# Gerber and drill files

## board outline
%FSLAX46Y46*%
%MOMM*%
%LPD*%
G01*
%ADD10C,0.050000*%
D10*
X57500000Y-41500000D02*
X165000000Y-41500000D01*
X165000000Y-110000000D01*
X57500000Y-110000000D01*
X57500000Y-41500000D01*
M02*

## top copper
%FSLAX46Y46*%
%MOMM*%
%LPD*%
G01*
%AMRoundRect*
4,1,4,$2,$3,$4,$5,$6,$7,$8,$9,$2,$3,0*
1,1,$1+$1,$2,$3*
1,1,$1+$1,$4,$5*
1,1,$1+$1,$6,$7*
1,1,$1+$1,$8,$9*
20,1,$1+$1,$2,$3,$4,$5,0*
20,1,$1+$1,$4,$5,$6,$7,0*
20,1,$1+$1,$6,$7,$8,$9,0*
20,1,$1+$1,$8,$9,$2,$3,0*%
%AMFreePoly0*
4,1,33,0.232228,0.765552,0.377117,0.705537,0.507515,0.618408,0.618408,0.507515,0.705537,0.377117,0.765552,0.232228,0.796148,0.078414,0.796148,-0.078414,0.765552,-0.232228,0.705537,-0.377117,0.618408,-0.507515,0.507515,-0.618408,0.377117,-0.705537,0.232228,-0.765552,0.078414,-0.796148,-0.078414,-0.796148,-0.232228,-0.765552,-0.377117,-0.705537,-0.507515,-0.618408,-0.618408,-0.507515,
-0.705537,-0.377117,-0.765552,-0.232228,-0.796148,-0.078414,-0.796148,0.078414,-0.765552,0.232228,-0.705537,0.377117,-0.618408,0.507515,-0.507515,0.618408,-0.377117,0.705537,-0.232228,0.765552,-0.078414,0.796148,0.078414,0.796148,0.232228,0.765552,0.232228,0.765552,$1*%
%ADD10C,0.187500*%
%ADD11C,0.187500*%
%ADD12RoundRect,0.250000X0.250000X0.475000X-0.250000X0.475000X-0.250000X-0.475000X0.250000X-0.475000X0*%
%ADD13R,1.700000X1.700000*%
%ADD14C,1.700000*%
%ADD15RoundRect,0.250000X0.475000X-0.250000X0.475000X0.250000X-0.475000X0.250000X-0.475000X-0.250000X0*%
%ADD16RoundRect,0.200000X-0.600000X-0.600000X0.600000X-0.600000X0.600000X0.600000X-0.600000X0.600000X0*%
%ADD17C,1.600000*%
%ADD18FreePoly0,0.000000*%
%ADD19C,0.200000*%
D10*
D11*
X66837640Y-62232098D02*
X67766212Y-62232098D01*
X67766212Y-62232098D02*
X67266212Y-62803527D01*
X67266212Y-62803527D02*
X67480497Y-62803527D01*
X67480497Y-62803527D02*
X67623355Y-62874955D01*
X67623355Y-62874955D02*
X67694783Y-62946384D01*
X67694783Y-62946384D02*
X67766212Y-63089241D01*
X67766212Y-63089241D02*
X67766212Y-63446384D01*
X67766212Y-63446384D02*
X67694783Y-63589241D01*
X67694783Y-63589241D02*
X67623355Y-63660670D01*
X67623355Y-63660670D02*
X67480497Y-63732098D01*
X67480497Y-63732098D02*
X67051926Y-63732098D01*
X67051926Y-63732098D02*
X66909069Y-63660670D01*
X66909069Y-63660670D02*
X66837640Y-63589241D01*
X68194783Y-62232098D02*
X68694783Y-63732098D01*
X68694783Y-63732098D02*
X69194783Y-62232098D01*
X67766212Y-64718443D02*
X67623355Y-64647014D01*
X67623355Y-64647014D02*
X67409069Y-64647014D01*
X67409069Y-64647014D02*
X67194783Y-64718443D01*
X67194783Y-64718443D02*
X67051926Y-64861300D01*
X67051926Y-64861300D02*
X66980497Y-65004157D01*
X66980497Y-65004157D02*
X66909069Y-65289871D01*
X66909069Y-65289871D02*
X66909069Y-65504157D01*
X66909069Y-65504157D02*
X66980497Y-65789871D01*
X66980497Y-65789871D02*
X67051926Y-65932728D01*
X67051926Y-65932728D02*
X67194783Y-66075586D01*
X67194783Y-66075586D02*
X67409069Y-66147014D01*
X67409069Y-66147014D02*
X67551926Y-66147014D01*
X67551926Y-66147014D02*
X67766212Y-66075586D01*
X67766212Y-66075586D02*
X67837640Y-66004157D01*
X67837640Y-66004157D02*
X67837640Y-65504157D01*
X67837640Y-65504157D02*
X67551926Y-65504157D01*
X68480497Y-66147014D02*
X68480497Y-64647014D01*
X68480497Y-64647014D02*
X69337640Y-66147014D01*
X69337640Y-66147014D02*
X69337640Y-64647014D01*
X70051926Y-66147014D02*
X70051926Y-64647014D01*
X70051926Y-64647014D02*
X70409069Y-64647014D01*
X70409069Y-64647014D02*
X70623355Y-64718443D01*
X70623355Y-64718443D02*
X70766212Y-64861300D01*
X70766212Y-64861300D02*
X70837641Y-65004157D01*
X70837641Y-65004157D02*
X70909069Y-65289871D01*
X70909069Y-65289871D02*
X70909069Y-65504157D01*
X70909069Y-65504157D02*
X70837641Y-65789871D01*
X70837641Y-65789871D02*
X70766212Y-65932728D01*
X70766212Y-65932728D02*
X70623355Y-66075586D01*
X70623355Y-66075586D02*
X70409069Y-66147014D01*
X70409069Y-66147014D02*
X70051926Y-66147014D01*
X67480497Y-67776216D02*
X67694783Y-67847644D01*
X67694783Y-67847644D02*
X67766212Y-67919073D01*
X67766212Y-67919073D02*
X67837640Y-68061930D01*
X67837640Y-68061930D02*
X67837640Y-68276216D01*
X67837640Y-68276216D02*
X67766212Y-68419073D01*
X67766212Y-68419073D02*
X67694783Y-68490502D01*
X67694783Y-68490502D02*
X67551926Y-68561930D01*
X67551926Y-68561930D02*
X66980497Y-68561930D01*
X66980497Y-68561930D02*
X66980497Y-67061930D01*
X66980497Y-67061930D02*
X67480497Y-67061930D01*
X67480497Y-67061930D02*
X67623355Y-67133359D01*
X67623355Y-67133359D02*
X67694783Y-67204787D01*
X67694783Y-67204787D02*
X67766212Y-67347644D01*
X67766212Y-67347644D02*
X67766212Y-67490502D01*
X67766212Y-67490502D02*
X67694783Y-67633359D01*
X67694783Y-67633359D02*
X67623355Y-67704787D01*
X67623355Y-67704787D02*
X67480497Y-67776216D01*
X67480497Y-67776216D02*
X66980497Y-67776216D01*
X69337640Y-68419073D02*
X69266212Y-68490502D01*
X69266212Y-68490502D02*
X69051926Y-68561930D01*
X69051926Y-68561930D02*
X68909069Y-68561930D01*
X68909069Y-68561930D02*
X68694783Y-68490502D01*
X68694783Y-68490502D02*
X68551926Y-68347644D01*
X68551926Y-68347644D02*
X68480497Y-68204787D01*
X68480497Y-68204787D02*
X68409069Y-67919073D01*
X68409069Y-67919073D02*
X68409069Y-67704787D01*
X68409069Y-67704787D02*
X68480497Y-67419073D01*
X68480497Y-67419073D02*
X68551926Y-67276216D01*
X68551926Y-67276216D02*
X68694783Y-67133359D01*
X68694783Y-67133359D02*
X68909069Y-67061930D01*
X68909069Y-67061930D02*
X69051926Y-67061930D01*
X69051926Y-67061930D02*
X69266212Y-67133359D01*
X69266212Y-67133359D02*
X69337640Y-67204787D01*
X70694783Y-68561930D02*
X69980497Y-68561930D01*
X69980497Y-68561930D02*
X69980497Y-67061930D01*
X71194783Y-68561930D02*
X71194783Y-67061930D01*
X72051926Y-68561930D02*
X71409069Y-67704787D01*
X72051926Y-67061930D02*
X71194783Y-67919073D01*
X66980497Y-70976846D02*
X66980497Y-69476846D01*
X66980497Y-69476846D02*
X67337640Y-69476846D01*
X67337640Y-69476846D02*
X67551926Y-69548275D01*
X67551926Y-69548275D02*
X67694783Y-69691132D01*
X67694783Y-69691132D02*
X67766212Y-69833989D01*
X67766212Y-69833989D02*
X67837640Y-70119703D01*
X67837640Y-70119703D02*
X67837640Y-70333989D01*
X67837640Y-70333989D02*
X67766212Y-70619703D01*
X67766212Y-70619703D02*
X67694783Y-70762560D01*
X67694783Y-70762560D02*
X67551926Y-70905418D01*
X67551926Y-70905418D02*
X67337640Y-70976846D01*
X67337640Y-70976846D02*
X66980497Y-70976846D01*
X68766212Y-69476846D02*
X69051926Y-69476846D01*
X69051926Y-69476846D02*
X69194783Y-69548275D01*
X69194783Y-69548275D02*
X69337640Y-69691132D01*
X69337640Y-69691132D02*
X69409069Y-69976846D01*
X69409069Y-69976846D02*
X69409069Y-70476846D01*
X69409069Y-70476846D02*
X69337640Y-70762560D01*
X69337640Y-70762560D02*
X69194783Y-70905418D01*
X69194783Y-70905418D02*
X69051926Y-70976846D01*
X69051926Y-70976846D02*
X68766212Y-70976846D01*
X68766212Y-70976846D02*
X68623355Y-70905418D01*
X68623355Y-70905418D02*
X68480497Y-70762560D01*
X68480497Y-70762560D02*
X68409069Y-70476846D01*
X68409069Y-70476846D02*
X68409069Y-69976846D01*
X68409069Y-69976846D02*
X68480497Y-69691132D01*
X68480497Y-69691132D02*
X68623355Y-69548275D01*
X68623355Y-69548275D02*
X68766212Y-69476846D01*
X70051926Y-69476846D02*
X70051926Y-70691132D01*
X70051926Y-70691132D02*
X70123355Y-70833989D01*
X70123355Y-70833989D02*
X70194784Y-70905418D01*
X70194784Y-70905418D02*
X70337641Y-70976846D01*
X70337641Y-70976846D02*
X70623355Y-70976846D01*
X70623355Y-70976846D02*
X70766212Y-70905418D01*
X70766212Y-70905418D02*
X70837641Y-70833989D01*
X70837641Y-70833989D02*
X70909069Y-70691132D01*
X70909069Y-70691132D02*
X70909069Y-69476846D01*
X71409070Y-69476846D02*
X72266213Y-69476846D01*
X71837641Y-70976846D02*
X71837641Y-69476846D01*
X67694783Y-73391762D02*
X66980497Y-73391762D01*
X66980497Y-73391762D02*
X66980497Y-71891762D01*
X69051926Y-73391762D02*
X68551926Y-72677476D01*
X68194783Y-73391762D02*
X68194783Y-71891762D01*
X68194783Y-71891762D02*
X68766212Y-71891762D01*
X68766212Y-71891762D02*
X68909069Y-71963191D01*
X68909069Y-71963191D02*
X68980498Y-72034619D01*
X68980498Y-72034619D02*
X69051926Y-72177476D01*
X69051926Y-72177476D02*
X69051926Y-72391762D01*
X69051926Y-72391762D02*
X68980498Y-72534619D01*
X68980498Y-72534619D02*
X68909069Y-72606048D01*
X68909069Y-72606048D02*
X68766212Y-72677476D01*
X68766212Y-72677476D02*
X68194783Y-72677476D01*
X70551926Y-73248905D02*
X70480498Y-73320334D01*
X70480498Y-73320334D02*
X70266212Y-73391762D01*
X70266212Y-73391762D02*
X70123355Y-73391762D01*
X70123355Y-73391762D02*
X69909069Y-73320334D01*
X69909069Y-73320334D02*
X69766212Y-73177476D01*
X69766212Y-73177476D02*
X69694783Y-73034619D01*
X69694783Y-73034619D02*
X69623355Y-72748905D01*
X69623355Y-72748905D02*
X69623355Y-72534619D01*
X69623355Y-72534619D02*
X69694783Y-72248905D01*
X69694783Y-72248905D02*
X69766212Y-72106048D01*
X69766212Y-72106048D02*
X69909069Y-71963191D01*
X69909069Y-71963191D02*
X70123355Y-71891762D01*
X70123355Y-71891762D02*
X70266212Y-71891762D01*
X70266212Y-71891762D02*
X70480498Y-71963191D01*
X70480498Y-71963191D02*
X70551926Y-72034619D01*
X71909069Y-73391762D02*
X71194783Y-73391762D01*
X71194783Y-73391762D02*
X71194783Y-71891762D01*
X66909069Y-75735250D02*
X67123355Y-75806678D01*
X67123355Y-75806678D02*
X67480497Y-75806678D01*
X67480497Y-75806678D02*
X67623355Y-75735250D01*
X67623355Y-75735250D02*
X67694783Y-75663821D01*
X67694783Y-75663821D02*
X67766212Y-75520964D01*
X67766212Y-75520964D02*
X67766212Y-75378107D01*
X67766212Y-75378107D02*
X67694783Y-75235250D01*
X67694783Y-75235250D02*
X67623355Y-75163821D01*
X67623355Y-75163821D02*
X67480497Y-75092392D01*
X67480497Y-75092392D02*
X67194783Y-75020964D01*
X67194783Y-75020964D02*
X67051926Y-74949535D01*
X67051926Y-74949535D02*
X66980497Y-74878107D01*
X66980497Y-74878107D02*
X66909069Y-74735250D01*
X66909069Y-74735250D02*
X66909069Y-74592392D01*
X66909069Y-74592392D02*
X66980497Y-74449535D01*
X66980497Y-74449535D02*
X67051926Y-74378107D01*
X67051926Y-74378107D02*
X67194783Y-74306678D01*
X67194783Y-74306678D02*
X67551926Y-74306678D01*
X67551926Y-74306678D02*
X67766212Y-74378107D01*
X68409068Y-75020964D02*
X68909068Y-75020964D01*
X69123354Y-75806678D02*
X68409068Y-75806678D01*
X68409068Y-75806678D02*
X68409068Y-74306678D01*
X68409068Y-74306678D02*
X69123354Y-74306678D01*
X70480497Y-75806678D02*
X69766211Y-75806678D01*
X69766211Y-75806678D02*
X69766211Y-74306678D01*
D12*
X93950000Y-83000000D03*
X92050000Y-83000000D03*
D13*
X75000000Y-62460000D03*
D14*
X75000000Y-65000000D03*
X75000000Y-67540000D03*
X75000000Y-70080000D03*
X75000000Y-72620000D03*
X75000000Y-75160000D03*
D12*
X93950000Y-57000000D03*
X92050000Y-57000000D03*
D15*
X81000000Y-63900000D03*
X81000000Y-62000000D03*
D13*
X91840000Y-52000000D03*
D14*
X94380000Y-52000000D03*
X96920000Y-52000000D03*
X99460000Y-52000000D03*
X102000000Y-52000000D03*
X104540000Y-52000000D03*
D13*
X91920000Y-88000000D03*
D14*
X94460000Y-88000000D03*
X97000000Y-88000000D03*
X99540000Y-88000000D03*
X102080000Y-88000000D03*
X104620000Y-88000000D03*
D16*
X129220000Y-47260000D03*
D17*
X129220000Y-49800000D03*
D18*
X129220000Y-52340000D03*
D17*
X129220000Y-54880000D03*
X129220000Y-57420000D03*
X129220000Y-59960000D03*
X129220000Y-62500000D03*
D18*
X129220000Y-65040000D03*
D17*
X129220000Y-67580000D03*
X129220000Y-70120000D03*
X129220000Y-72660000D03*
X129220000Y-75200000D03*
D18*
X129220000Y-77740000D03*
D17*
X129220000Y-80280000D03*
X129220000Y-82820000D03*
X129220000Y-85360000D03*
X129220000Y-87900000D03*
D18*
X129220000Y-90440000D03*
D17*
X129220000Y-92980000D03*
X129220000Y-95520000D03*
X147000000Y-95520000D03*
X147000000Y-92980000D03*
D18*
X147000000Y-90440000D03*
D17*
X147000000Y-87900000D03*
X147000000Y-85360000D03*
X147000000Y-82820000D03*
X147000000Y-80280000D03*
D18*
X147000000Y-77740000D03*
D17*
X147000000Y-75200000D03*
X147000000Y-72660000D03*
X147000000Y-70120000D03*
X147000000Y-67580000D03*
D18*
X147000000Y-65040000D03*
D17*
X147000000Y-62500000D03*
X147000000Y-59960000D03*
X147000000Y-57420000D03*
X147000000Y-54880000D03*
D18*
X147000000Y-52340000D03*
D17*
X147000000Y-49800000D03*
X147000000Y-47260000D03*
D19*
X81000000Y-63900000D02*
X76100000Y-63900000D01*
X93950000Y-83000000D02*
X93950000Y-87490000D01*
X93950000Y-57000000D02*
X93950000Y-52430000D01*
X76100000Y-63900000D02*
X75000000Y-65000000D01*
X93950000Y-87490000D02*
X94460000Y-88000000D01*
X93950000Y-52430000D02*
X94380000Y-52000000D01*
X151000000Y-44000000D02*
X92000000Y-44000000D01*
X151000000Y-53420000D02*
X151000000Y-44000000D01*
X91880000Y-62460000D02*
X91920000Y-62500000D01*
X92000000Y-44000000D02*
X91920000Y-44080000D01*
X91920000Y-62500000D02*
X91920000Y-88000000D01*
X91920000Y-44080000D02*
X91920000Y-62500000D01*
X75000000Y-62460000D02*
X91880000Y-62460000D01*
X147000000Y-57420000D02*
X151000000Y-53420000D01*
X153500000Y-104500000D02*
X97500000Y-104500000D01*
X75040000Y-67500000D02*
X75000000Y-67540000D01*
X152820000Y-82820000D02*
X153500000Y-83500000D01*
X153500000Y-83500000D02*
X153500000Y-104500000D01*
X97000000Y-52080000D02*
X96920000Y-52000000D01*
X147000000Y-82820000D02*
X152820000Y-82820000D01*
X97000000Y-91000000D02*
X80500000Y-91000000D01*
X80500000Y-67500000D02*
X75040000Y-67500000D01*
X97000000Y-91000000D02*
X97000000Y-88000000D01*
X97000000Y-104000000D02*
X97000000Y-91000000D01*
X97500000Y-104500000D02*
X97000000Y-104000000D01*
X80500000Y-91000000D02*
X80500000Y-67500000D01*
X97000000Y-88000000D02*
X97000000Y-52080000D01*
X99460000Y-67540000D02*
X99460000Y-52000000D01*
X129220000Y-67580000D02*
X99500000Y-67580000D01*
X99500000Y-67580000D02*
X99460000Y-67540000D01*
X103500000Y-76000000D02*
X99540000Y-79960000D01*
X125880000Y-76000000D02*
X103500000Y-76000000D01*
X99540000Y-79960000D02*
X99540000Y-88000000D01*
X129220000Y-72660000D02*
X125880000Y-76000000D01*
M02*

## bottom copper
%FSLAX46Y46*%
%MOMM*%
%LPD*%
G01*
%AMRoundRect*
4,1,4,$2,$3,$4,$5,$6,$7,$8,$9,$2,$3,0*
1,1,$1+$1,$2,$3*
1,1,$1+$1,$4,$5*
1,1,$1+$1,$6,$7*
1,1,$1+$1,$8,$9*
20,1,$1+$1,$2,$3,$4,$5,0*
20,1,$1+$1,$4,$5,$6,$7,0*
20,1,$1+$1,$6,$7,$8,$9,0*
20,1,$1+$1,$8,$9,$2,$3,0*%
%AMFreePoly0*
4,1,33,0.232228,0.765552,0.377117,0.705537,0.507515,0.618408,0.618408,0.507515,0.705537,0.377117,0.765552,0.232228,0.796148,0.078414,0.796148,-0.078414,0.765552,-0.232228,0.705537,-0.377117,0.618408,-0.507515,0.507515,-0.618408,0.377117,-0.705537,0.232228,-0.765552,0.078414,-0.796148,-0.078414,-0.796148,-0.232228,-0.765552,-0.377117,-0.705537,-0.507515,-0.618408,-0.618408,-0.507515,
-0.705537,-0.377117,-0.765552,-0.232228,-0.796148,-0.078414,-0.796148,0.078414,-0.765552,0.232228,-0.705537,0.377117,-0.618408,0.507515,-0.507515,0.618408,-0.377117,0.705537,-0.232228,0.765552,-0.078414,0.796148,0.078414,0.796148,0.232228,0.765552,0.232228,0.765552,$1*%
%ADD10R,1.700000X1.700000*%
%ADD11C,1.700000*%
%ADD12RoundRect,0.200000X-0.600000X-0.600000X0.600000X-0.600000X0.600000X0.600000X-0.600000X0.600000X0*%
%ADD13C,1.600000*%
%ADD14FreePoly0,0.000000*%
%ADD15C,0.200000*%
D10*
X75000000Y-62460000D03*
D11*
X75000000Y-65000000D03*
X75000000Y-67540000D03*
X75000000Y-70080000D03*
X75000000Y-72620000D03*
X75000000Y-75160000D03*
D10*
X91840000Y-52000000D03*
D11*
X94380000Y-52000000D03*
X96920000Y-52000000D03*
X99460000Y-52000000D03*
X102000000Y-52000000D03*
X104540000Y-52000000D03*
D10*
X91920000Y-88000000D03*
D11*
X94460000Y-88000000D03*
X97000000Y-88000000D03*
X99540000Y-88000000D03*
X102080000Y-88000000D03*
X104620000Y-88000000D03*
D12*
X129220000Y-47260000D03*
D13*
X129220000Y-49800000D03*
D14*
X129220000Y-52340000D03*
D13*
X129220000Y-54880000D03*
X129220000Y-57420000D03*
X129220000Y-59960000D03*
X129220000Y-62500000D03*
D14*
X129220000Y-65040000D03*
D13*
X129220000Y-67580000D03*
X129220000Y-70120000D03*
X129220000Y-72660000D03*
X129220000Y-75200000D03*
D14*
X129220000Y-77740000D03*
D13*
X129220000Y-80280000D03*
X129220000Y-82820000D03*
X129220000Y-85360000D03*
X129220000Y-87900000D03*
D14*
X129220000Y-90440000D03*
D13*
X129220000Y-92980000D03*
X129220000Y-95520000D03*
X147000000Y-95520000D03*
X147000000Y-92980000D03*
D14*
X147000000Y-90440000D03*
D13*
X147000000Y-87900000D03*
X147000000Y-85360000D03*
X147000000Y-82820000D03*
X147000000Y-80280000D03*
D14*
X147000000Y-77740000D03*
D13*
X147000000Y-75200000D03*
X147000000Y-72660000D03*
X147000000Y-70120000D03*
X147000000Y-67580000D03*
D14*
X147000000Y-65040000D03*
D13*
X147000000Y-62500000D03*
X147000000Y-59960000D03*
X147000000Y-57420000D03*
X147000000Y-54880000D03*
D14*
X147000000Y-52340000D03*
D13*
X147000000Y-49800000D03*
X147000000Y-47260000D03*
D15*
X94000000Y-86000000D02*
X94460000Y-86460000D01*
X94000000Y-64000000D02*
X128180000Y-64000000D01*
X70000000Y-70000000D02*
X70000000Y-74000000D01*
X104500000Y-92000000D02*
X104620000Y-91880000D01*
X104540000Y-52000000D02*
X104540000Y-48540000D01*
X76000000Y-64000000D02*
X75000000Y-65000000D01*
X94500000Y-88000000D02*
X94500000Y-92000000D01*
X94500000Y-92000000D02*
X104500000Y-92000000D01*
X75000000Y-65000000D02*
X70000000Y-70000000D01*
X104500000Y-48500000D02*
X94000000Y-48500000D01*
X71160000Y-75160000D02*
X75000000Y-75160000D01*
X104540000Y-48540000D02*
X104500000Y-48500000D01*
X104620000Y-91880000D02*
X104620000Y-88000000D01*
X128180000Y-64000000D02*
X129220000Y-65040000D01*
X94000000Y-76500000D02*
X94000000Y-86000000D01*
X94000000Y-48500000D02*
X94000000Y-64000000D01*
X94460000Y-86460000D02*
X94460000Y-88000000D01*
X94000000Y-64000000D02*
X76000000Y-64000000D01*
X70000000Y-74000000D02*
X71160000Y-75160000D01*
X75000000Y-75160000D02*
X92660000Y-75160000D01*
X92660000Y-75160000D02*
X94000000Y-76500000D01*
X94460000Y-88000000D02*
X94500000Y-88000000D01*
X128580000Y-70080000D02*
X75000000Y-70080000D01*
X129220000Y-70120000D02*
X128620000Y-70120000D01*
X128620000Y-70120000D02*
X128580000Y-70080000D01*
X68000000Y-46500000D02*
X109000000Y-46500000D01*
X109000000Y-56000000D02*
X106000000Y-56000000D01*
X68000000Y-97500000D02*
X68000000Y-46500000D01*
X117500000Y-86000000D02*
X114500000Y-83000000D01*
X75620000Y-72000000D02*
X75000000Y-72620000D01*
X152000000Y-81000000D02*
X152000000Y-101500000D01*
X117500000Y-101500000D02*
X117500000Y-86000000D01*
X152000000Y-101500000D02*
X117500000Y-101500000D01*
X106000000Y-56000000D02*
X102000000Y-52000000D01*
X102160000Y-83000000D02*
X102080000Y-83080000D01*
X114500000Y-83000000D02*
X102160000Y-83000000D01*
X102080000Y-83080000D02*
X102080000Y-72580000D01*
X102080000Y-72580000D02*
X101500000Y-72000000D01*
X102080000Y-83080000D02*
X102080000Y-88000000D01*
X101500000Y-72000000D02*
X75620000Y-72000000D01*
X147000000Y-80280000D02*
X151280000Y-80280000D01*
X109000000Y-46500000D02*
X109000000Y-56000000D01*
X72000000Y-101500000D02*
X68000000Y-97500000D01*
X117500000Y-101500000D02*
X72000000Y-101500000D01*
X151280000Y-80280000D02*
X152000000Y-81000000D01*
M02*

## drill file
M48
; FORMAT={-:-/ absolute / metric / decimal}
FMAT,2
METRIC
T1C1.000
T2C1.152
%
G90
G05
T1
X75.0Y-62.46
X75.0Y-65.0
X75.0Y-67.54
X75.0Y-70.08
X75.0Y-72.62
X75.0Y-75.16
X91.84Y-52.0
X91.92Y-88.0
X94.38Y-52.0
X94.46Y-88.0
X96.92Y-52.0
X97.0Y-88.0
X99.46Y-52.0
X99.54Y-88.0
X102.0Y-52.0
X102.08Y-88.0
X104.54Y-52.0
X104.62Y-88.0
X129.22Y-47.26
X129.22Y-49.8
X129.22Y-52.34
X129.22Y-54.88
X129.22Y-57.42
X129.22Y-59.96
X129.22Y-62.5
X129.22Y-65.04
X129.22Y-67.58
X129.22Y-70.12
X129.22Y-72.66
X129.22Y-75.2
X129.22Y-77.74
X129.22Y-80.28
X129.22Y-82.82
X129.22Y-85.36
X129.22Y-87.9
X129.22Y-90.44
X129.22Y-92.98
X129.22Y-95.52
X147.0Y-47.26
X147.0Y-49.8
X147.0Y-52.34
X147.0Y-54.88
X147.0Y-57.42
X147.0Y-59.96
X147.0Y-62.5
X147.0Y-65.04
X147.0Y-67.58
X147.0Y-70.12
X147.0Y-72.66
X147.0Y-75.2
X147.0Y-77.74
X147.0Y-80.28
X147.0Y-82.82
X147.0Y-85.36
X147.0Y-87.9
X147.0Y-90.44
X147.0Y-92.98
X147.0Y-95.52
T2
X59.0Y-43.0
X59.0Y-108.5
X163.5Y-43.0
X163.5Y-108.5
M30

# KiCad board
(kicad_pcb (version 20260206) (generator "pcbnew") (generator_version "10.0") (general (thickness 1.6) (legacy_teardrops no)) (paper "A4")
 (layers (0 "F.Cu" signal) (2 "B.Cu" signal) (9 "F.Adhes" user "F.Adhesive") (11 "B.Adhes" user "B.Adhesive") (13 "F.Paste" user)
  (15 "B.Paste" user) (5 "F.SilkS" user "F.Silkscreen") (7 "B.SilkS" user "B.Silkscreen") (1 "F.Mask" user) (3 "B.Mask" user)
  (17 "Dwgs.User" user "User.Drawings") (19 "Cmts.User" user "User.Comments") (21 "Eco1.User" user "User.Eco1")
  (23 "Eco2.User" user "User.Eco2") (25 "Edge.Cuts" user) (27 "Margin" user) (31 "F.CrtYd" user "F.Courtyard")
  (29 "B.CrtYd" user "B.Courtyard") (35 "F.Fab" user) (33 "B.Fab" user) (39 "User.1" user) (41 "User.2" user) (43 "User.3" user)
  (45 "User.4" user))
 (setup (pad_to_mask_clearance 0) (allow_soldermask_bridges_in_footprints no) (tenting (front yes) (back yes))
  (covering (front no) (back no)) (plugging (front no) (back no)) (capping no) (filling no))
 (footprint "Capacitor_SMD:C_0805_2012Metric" (layer "F.Cu") (at 93 83 180)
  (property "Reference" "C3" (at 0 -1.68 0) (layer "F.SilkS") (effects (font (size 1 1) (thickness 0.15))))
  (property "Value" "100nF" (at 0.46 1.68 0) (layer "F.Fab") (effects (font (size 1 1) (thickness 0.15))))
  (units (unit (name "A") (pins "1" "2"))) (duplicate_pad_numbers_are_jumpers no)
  (pad "1" smd roundrect (at -0.95 0 180) (size 1 1.45) (layers "F.Cu" "F.Mask" "F.Paste") (roundrect_rratio 0.25) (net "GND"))
  (pad "2" smd roundrect (at 0.95 0 180) (size 1 1.45) (layers "F.Cu" "F.Mask" "F.Paste") (roundrect_rratio 0.25) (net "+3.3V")))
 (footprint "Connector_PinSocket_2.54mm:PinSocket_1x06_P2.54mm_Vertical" (layer "F.Cu") (at 75 62.46)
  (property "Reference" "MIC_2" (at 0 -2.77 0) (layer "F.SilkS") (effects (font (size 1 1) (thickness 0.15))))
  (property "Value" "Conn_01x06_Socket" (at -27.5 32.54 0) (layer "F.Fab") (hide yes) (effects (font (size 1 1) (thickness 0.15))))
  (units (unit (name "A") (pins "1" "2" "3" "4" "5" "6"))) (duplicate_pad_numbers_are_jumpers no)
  (pad "1" thru_hole rect (at 0 0) (size 1.7 1.7) (drill 1) (layers "*.Cu" "*.Mask") (remove_unused_layers no) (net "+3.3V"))
  (pad "2" thru_hole circle (at 0 2.54) (size 1.7 1.7) (drill 1) (layers "*.Cu" "*.Mask") (remove_unused_layers no) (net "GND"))
  (pad "3" thru_hole circle (at 0 5.08) (size 1.7 1.7) (drill 1) (layers "*.Cu" "*.Mask") (remove_unused_layers no) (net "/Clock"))
  (pad "4" thru_hole circle (at 0 7.62) (size 1.7 1.7) (drill 1) (layers "*.Cu" "*.Mask") (remove_unused_layers no) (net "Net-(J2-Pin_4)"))
  (pad "5" thru_hole circle (at 0 10.16) (size 1.7 1.7) (drill 1) (layers "*.Cu" "*.Mask") (remove_unused_layers no) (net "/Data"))
  (pad "6" thru_hole circle (at 0 12.7) (size 1.7 1.7) (drill 1) (layers "*.Cu" "*.Mask") (remove_unused_layers no) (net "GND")))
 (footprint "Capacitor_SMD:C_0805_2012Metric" (layer "F.Cu") (at 93 57 180)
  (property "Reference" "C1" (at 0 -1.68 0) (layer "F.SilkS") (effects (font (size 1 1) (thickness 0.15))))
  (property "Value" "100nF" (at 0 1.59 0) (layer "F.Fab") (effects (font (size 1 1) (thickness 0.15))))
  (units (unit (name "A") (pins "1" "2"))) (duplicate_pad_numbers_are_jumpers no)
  (pad "1" smd roundrect (at -0.95 0 180) (size 1 1.45) (layers "F.Cu" "F.Mask" "F.Paste") (roundrect_rratio 0.25) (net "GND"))
  (pad "2" smd roundrect (at 0.95 0 180) (size 1 1.45) (layers "F.Cu" "F.Mask" "F.Paste") (roundrect_rratio 0.25) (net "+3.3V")))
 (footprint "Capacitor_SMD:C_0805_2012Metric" (layer "F.Cu") (at 81 62.95 90)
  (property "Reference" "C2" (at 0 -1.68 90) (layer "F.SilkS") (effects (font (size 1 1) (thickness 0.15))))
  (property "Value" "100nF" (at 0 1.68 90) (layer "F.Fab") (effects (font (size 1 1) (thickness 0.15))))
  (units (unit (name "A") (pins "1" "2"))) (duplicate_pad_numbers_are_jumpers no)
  (pad "1" smd roundrect (at -0.95 0 90) (size 1 1.45) (layers "F.Cu" "F.Mask" "F.Paste") (roundrect_rratio 0.25) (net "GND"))
  (pad "2" smd roundrect (at 0.95 0 90) (size 1 1.45) (layers "F.Cu" "F.Mask" "F.Paste") (roundrect_rratio 0.25) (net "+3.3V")))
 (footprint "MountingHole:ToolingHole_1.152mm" (layer "F.Cu") (at 59 43)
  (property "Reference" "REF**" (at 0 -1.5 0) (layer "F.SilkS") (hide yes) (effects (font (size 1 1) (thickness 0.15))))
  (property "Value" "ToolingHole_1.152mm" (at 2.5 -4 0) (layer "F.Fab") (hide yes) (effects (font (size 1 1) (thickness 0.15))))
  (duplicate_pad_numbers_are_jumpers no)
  (pad "" np_thru_hole circle (at 0 0) (size 1.152 1.152) (drill 1.152) (layers "*.Cu" "*.Mask") (solder_mask_margin 0.074))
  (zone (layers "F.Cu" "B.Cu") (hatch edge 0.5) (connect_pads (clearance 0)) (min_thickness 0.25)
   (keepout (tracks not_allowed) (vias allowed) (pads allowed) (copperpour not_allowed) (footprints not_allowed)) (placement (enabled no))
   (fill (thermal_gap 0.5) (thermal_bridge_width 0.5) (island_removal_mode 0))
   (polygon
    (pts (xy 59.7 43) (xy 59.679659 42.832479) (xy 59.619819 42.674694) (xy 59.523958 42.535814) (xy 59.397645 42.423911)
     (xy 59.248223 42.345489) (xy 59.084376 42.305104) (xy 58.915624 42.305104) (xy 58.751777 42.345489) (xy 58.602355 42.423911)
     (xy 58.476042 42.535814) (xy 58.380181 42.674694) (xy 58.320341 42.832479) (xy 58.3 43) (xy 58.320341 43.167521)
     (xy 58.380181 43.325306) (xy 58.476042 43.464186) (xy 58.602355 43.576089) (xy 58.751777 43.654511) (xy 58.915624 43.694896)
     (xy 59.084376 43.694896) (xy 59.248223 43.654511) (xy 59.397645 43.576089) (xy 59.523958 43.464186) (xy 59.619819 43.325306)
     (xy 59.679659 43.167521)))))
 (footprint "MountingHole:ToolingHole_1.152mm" (layer "F.Cu") (at 163.5 108.5)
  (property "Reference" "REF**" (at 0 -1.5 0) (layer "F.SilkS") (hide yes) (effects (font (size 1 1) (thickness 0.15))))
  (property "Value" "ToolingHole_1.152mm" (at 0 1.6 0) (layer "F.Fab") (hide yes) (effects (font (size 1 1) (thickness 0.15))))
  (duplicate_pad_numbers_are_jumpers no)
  (pad "" np_thru_hole circle (at 0 0) (size 1.152 1.152) (drill 1.152) (layers "*.Cu" "*.Mask") (solder_mask_margin 0.074))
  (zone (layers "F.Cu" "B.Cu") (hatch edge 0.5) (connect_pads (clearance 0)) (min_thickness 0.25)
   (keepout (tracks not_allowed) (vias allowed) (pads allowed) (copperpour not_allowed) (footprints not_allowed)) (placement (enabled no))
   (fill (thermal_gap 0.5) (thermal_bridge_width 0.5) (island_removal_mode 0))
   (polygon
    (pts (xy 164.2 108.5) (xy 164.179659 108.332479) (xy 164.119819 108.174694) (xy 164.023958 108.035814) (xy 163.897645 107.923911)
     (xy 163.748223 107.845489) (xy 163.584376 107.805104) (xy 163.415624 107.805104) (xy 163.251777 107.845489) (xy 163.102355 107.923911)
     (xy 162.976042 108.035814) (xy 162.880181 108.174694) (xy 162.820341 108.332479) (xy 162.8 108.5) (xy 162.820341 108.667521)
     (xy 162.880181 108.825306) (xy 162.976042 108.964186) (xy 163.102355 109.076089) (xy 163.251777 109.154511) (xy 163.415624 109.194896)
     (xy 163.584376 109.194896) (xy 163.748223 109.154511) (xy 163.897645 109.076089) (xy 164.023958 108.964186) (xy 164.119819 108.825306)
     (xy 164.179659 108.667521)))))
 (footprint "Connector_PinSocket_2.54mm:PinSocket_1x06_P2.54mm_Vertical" (layer "F.Cu") (at 91.84 52 90)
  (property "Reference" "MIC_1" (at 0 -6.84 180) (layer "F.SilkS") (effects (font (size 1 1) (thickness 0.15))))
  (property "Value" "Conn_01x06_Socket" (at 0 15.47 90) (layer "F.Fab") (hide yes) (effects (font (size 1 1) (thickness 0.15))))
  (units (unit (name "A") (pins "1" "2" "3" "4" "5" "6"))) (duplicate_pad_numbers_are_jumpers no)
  (pad "1" thru_hole rect (at 0 0 90) (size 1.7 1.7) (drill 1) (layers "*.Cu" "*.Mask") (remove_unused_layers no) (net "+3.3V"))
  (pad "2" thru_hole circle (at 0 2.54 90) (size 1.7 1.7) (drill 1) (layers "*.Cu" "*.Mask") (remove_unused_layers no) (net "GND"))
  (pad "3" thru_hole circle (at 0 5.08 90) (size 1.7 1.7) (drill 1) (layers "*.Cu" "*.Mask") (remove_unused_layers no) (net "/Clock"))
  (pad "4" thru_hole circle (at 0 7.62 90) (size 1.7 1.7) (drill 1) (layers "*.Cu" "*.Mask") (remove_unused_layers no)
   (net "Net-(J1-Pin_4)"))
  (pad "5" thru_hole circle (at 0 10.16 90) (size 1.7 1.7) (drill 1) (layers "*.Cu" "*.Mask") (remove_unused_layers no) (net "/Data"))
  (pad "6" thru_hole circle (at 0 12.7 90) (size 1.7 1.7) (drill 1) (layers "*.Cu" "*.Mask") (remove_unused_layers no) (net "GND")))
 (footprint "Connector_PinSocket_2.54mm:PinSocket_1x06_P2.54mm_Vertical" (layer "F.Cu") (at 91.92 88 90)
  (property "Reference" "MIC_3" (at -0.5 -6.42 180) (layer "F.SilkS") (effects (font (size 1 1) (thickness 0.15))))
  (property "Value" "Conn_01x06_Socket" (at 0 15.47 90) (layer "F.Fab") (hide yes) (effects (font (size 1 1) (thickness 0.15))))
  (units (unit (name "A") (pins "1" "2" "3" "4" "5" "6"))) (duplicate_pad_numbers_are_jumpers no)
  (pad "1" thru_hole rect (at 0 0 90) (size 1.7 1.7) (drill 1) (layers "*.Cu" "*.Mask") (remove_unused_layers no) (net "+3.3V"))
  (pad "2" thru_hole circle (at 0 2.54 90) (size 1.7 1.7) (drill 1) (layers "*.Cu" "*.Mask") (remove_unused_layers no) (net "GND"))
  (pad "3" thru_hole circle (at 0 5.08 90) (size 1.7 1.7) (drill 1) (layers "*.Cu" "*.Mask") (remove_unused_layers no) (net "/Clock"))
  (pad "4" thru_hole circle (at 0 7.62 90) (size 1.7 1.7) (drill 1) (layers "*.Cu" "*.Mask") (remove_unused_layers no)
   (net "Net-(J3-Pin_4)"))
  (pad "5" thru_hole circle (at 0 10.16 90) (size 1.7 1.7) (drill 1) (layers "*.Cu" "*.Mask") (remove_unused_layers no) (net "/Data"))
  (pad "6" thru_hole circle (at 0 12.7 90) (size 1.7 1.7) (drill 1) (layers "*.Cu" "*.Mask") (remove_unused_layers no) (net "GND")))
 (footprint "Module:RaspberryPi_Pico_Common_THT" (layer "F.Cu") (at 129.22 47.26)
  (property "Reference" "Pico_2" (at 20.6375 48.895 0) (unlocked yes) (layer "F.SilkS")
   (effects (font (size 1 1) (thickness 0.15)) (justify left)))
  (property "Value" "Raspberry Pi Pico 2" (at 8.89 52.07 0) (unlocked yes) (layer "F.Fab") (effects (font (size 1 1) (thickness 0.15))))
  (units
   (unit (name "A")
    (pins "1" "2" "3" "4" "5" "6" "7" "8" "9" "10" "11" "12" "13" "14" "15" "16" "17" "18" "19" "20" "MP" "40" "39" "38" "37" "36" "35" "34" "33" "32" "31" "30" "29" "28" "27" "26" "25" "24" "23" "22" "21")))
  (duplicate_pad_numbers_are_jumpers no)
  (pad "1" thru_hole roundrect (at 0 0) (size 1.6 1.6) (drill 1) (layers "*.Cu" "*.Mask") (remove_unused_layers no) (roundrect_rratio 0.125)
   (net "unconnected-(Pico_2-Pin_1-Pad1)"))
  (pad "2" thru_hole circle (at 0 2.54) (size 1.6 1.6) (drill 1) (layers "*.Cu" "*.Mask") (remove_unused_layers no)
   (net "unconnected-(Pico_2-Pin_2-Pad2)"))
  (pad "3" thru_hole custom (at 0 5.08) (size 1.6 1.6) (drill 1) (layers "*.Cu" "*.Mask") (remove_unused_layers no)
   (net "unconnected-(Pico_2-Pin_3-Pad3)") (options (clearance outline) (anchor circle)) (primitives))
  (pad "4" thru_hole circle (at 0 7.62) (size 1.6 1.6) (drill 1) (layers "*.Cu" "*.Mask") (remove_unused_layers no)
   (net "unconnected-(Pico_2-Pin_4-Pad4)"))
  (pad "5" thru_hole circle (at 0 10.16) (size 1.6 1.6) (drill 1) (layers "*.Cu" "*.Mask") (remove_unused_layers no)
   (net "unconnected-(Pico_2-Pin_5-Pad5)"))
  (pad "6" thru_hole circle (at 0 12.7) (size 1.6 1.6) (drill 1) (layers "*.Cu" "*.Mask") (remove_unused_layers no)
   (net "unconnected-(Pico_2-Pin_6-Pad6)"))
  (pad "7" thru_hole circle (at 0 15.24) (size 1.6 1.6) (drill 1) (layers "*.Cu" "*.Mask") (remove_unused_layers no)
   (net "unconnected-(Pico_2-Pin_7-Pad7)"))
  (pad "8" thru_hole custom (at 0 17.78) (size 1.6 1.6) (drill 1) (layers "*.Cu" "*.Mask") (remove_unused_layers no) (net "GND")
   (options (clearance outline) (anchor circle)) (primitives))
  (pad "9" thru_hole circle (at 0 20.32) (size 1.6 1.6) (drill 1) (layers "*.Cu" "*.Mask") (remove_unused_layers no) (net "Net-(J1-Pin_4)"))
  (pad "10" thru_hole circle (at 0 22.86) (size 1.6 1.6) (drill 1) (layers "*.Cu" "*.Mask") (remove_unused_layers no) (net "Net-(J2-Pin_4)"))
  (pad "11" thru_hole circle (at 0 25.4) (size 1.6 1.6) (drill 1) (layers "*.Cu" "*.Mask") (remove_unused_layers no) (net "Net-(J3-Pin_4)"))
  (pad "12" thru_hole circle (at 0 27.94) (size 1.6 1.6) (drill 1) (layers "*.Cu" "*.Mask") (remove_unused_layers no)
   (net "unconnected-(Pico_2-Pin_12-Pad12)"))
  (pad "13" thru_hole custom (at 0 30.48) (size 1.6 1.6) (drill 1) (layers "*.Cu" "*.Mask") (remove_unused_layers no)
   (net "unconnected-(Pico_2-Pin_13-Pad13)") (options (clearance outline) (anchor circle)) (primitives))
  (pad "14" thru_hole circle (at 0 33.02) (size 1.6 1.6) (drill 1) (layers "*.Cu" "*.Mask") (remove_unused_layers no)
   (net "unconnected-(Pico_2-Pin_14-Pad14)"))
  (pad "15" thru_hole circle (at 0 35.56) (size 1.6 1.6) (drill 1) (layers "*.Cu" "*.Mask") (remove_unused_layers no)
   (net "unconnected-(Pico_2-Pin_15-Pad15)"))
  (pad "16" thru_hole circle (at 0 38.1) (size 1.6 1.6) (drill 1) (layers "*.Cu" "*.Mask") (remove_unused_layers no)
   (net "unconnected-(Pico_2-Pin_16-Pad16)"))
  (pad "17" thru_hole circle (at 0 40.64) (size 1.6 1.6) (drill 1) (layers "*.Cu" "*.Mask") (remove_unused_layers no)
   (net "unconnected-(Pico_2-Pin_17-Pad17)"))
  (pad "18" thru_hole custom (at 0 43.18) (size 1.6 1.6) (drill 1) (layers "*.Cu" "*.Mask") (remove_unused_layers no)
   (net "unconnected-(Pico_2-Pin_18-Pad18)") (options (clearance outline) (anchor circle)) (primitives))
  (pad "19" thru_hole circle (at 0 45.72) (size 1.6 1.6) (drill 1) (layers "*.Cu" "*.Mask") (remove_unused_layers no)
   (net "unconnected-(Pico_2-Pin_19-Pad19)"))
  (pad "20" thru_hole circle (at 0 48.26) (size 1.6 1.6) (drill 1) (layers "*.Cu" "*.Mask") (remove_unused_layers no)
   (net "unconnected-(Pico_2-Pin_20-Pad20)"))
  (pad "21" thru_hole circle (at 17.78 48.26) (size 1.6 1.6) (drill 1) (layers "*.Cu" "*.Mask") (remove_unused_layers no)
   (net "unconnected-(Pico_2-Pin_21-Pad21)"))
  (pad "22" thru_hole circle (at 17.78 45.72) (size 1.6 1.6) (drill 1) (layers "*.Cu" "*.Mask") (remove_unused_layers no)
   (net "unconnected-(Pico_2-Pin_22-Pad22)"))
  (pad "23" thru_hole custom (at 17.78 43.18) (size 1.6 1.6) (drill 1) (layers "*.Cu" "*.Mask") (remove_unused_layers no)
   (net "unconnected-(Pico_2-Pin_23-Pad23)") (options (clearance outline) (anchor circle)) (primitives))
  (pad "24" thru_hole circle (at 17.78 40.64) (size 1.6 1.6) (drill 1) (layers "*.Cu" "*.Mask") (remove_unused_layers no)
   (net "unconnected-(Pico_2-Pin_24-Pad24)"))
  (pad "25" thru_hole circle (at 17.78 38.1) (size 1.6 1.6) (drill 1) (layers "*.Cu" "*.Mask") (remove_unused_layers no)
   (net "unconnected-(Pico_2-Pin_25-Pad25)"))
  (pad "26" thru_hole circle (at 17.78 35.56) (size 1.6 1.6) (drill 1) (layers "*.Cu" "*.Mask") (remove_unused_layers no) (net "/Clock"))
  (pad "27" thru_hole circle (at 17.78 33.02) (size 1.6 1.6) (drill 1) (layers "*.Cu" "*.Mask") (remove_unused_layers no) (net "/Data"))
  (pad "28" thru_hole custom (at 17.78 30.48) (size 1.6 1.6) (drill 1) (layers "*.Cu" "*.Mask") (remove_unused_layers no)
   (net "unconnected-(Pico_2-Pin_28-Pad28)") (options (clearance outline) (anchor circle)) (primitives))
  (pad "29" thru_hole circle (at 17.78 27.94) (size 1.6 1.6) (drill 1) (layers "*.Cu" "*.Mask") (remove_unused_layers no)
   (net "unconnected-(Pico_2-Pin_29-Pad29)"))
  (pad "30" thru_hole circle (at 17.78 25.4) (size 1.6 1.6) (drill 1) (layers "*.Cu" "*.Mask") (remove_unused_layers no)
   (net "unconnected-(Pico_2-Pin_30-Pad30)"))
  (pad "31" thru_hole circle (at 17.78 22.86) (size 1.6 1.6) (drill 1) (layers "*.Cu" "*.Mask") (remove_unused_layers no)
   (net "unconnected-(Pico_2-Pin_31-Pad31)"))
  (pad "32" thru_hole circle (at 17.78 20.32) (size 1.6 1.6) (drill 1) (layers "*.Cu" "*.Mask") (remove_unused_layers no)
   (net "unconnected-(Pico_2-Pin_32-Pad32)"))
  (pad "33" thru_hole custom (at 17.78 17.78) (size 1.6 1.6) (drill 1) (layers "*.Cu" "*.Mask") (remove_unused_layers no)
   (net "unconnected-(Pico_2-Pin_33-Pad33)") (options (clearance outline) (anchor circle)) (primitives))
  (pad "34" thru_hole circle (at 17.78 15.24) (size 1.6 1.6) (drill 1) (layers "*.Cu" "*.Mask") (remove_unused_layers no)
   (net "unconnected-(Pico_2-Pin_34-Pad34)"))
  (pad "35" thru_hole circle (at 17.78 12.7) (size 1.6 1.6) (drill 1) (layers "*.Cu" "*.Mask") (remove_unused_layers no)
   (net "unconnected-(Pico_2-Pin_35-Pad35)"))
  (pad "36" thru_hole circle (at 17.78 10.16) (size 1.6 1.6) (drill 1) (layers "*.Cu" "*.Mask") (remove_unused_layers no) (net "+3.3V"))
  (pad "37" thru_hole circle (at 17.78 7.62) (size 1.6 1.6) (drill 1) (layers "*.Cu" "*.Mask") (remove_unused_layers no)
   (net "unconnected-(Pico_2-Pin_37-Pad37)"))
  (pad "38" thru_hole custom (at 17.78 5.08) (size 1.6 1.6) (drill 1) (layers "*.Cu" "*.Mask") (remove_unused_layers no)
   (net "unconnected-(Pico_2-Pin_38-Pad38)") (options (clearance outline) (anchor circle)) (primitives))
  (pad "39" thru_hole circle (at 17.78 2.54) (size 1.6 1.6) (drill 1) (layers "*.Cu" "*.Mask") (remove_unused_layers no)
   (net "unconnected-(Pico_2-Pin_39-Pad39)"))
  (pad "40" thru_hole circle (at 17.78 0) (size 1.6 1.6) (drill 1) (layers "*.Cu" "*.Mask") (remove_unused_layers no)
   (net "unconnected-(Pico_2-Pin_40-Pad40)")))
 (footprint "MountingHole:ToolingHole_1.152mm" (layer "F.Cu") (at 59 108.5)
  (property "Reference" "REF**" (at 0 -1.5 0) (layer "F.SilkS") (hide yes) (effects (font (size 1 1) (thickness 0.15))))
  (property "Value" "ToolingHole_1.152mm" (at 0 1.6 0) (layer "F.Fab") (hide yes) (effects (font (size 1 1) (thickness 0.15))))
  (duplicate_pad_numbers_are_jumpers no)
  (pad "" np_thru_hole circle (at 0 0) (size 1.152 1.152) (drill 1.152) (layers "*.Cu" "*.Mask") (solder_mask_margin 0.074))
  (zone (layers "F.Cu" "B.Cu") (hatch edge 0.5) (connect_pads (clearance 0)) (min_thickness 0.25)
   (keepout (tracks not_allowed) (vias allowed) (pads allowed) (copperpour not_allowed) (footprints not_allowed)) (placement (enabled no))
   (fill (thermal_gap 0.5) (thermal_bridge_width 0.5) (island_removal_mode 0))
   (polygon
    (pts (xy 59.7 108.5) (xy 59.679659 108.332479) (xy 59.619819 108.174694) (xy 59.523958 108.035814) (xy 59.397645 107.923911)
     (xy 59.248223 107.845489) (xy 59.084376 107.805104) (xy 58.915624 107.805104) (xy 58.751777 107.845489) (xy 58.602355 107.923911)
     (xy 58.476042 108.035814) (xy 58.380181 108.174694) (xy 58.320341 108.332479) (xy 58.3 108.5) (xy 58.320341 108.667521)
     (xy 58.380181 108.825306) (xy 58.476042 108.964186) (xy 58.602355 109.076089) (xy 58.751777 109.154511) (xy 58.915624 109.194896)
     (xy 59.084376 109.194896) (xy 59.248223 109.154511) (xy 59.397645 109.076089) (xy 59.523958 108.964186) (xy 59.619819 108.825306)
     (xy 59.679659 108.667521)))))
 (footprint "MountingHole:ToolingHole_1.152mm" (layer "F.Cu") (at 163.5 43)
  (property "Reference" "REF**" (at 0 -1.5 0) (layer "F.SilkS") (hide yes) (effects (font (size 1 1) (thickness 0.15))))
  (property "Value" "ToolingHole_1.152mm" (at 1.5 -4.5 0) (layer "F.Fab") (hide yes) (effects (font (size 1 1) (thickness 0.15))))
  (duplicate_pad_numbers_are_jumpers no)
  (pad "" np_thru_hole circle (at 0 0) (size 1.152 1.152) (drill 1.152) (layers "*.Cu" "*.Mask") (solder_mask_margin 0.074))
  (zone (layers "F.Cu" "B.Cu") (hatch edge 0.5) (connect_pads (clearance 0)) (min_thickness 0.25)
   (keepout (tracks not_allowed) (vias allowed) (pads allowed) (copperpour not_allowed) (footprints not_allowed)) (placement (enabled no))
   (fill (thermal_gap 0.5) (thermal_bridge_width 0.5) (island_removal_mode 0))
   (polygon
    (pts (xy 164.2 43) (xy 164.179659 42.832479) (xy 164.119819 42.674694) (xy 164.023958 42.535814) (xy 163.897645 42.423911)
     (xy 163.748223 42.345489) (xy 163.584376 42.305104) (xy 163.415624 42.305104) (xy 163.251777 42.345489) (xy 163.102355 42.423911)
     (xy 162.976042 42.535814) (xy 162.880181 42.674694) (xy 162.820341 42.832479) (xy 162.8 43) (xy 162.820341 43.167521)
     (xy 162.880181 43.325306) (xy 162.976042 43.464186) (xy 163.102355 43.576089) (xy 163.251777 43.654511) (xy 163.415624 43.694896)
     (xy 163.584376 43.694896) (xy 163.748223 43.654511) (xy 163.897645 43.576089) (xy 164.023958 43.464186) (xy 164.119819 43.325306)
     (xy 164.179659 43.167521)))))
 (gr_rect (start 57.5 41.5) (end 165 110) (stroke (width 0.05) (type default)) (fill no) (layer "Edge.Cuts"))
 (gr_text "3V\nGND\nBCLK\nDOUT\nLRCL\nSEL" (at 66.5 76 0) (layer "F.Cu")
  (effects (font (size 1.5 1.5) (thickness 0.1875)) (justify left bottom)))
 (segment (start 81 63.9) (end 76.1 63.9) (width 0.2) (layer "F.Cu") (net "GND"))
 (segment (start 93.95 83) (end 93.95 87.49) (width 0.2) (layer "F.Cu") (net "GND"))
 (segment (start 93.95 57) (end 93.95 52.43) (width 0.2) (layer "F.Cu") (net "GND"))
 (segment (start 76.1 63.9) (end 75 65) (width 0.2) (layer "F.Cu") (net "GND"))
 (segment (start 93.95 87.49) (end 94.46 88) (width 0.2) (layer "F.Cu") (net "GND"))
 (segment (start 93.95 52.43) (end 94.38 52) (width 0.2) (layer "F.Cu") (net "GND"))
 (segment (start 94 86) (end 94.46 86.46) (width 0.2) (layer "B.Cu") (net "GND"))
 (segment (start 94 64) (end 128.18 64) (width 0.2) (layer "B.Cu") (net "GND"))
 (segment (start 70 70) (end 70 74) (width 0.2) (layer "B.Cu") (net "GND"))
 (segment (start 104.5 92) (end 104.62 91.88) (width 0.2) (layer "B.Cu") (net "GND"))
 (segment (start 104.54 52) (end 104.54 48.54) (width 0.2) (layer "B.Cu") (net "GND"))
 (segment (start 76 64) (end 75 65) (width 0.2) (layer "B.Cu") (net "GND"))
 (segment (start 94.5 88) (end 94.5 92) (width 0.2) (layer "B.Cu") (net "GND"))
 (segment (start 94.5 92) (end 104.5 92) (width 0.2) (layer "B.Cu") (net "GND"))
 (segment (start 75 65) (end 70 70) (width 0.2) (layer "B.Cu") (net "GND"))
 (segment (start 104.5 48.5) (end 94 48.5) (width 0.2) (layer "B.Cu") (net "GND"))
 (segment (start 71.16 75.16) (end 75 75.16) (width 0.2) (layer "B.Cu") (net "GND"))
 (segment (start 104.54 48.54) (end 104.5 48.5) (width 0.2) (layer "B.Cu") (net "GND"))
 (segment (start 104.62 91.88) (end 104.62 88) (width 0.2) (layer "B.Cu") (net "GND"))
 (segment (start 128.18 64) (end 129.22 65.04) (width 0.2) (layer "B.Cu") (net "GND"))
 (segment (start 94 76.5) (end 94 86) (width 0.2) (layer "B.Cu") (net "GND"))
 (segment (start 94 48.5) (end 94 64) (width 0.2) (layer "B.Cu") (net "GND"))
 (segment (start 94.46 86.46) (end 94.46 88) (width 0.2) (layer "B.Cu") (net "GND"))
 (segment (start 94 64) (end 76 64) (width 0.2) (layer "B.Cu") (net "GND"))
 (segment (start 70 74) (end 71.16 75.16) (width 0.2) (layer "B.Cu") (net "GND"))
 (segment (start 75 75.16) (end 92.66 75.16) (width 0.2) (layer "B.Cu") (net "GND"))
 (segment (start 92.66 75.16) (end 94 76.5) (width 0.2) (layer "B.Cu") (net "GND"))
 (segment (start 94.46 88) (end 94.5 88) (width 0.2) (layer "B.Cu") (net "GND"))
 (segment (start 151 44) (end 92 44) (width 0.2) (layer "F.Cu") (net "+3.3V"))
 (segment (start 151 53.42) (end 151 44) (width 0.2) (layer "F.Cu") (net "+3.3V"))
 (segment (start 91.88 62.46) (end 91.92 62.5) (width 0.2) (layer "F.Cu") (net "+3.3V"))
 (segment (start 92 44) (end 91.92 44.08) (width 0.2) (layer "F.Cu") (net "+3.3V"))
 (segment (start 91.92 62.5) (end 91.92 88) (width 0.2) (layer "F.Cu") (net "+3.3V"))
 (segment (start 91.92 44.08) (end 91.92 62.5) (width 0.2) (layer "F.Cu") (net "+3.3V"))
 (segment (start 75 62.46) (end 91.88 62.46) (width 0.2) (layer "F.Cu") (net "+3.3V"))
 (segment (start 147 57.42) (end 151 53.42) (width 0.2) (layer "F.Cu") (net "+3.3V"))
 (segment (start 153.5 104.5) (end 97.5 104.5) (width 0.2) (layer "F.Cu") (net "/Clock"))
 (segment (start 75.04 67.5) (end 75 67.54) (width 0.2) (layer "F.Cu") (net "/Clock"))
 (segment (start 152.82 82.82) (end 153.5 83.5) (width 0.2) (layer "F.Cu") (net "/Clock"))
 (segment (start 153.5 83.5) (end 153.5 104.5) (width 0.2) (layer "F.Cu") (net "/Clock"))
 (segment (start 97 52.08) (end 96.92 52) (width 0.2) (layer "F.Cu") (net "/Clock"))
 (segment (start 147 82.82) (end 152.82 82.82) (width 0.2) (layer "F.Cu") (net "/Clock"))
 (segment (start 97 91) (end 80.5 91) (width 0.2) (layer "F.Cu") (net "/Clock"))
 (segment (start 80.5 67.5) (end 75.04 67.5) (width 0.2) (layer "F.Cu") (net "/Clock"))
 (segment (start 97 91) (end 97 88) (width 0.2) (layer "F.Cu") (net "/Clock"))
 (segment (start 97 104) (end 97 91) (width 0.2) (layer "F.Cu") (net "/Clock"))
 (segment (start 97.5 104.5) (end 97 104) (width 0.2) (layer "F.Cu") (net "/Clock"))
 (segment (start 80.5 91) (end 80.5 67.5) (width 0.2) (layer "F.Cu") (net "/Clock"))
 (segment (start 97 88) (end 97 52.08) (width 0.2) (layer "F.Cu") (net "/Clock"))
 (segment (start 128.58 70.08) (end 75 70.08) (width 0.2) (layer "B.Cu") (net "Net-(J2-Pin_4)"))
 (segment (start 129.22 70.12) (end 128.62 70.12) (width 0.2) (layer "B.Cu") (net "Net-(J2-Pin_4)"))
 (segment (start 128.62 70.12) (end 128.58 70.08) (width 0.2) (layer "B.Cu") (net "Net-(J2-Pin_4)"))
 (segment (start 68 46.5) (end 109 46.5) (width 0.2) (layer "B.Cu") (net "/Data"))
 (segment (start 109 56) (end 106 56) (width 0.2) (layer "B.Cu") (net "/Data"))
 (segment (start 68 97.5) (end 68 46.5) (width 0.2) (layer "B.Cu") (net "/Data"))
 (segment (start 117.5 86) (end 114.5 83) (width 0.2) (layer "B.Cu") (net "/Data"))
 (segment (start 75.62 72) (end 75 72.62) (width 0.2) (layer "B.Cu") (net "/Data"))
 (segment (start 152 81) (end 152 101.5) (width 0.2) (layer "B.Cu") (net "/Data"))
 (segment (start 117.5 101.5) (end 117.5 86) (width 0.2) (layer "B.Cu") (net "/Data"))
 (segment (start 152 101.5) (end 117.5 101.5) (width 0.2) (layer "B.Cu") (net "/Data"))
 (segment (start 106 56) (end 102 52) (width 0.2) (layer "B.Cu") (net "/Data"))
 (segment (start 102.16 83) (end 102.08 83.08) (width 0.2) (layer "B.Cu") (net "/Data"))
 (segment (start 114.5 83) (end 102.16 83) (width 0.2) (layer "B.Cu") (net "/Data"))
 (segment (start 102.08 83.08) (end 102.08 72.58) (width 0.2) (layer "B.Cu") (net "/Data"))
 (segment (start 102.08 72.58) (end 101.5 72) (width 0.2) (layer "B.Cu") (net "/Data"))
 (segment (start 102.08 83.08) (end 102.08 88) (width 0.2) (layer "B.Cu") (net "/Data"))
 (segment (start 101.5 72) (end 75.62 72) (width 0.2) (layer "B.Cu") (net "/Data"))
 (segment (start 147 80.28) (end 151.28 80.28) (width 0.2) (layer "B.Cu") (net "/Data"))
 (segment (start 109 46.5) (end 109 56) (width 0.2) (layer "B.Cu") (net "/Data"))
 (segment (start 72 101.5) (end 68 97.5) (width 0.2) (layer "B.Cu") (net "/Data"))
 (segment (start 117.5 101.5) (end 72 101.5) (width 0.2) (layer "B.Cu") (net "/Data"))
 (segment (start 151.28 80.28) (end 152 81) (width 0.2) (layer "B.Cu") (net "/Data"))
 (segment (start 99.46 67.54) (end 99.46 52) (width 0.2) (layer "F.Cu") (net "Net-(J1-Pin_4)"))
 (segment (start 129.22 67.58) (end 99.5 67.58) (width 0.2) (layer "F.Cu") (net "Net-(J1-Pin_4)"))
 (segment (start 99.5 67.58) (end 99.46 67.54) (width 0.2) (layer "F.Cu") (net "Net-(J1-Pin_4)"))
 (segment (start 103.5 76) (end 99.54 79.96) (width 0.2) (layer "F.Cu") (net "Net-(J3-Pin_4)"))
 (segment (start 125.88 76) (end 103.5 76) (width 0.2) (layer "F.Cu") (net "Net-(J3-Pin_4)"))
 (segment (start 99.54 79.96) (end 99.54 88) (width 0.2) (layer "F.Cu") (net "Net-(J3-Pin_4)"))
 (segment (start 129.22 72.66) (end 125.88 76) (width 0.2) (layer "F.Cu") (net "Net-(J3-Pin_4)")))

